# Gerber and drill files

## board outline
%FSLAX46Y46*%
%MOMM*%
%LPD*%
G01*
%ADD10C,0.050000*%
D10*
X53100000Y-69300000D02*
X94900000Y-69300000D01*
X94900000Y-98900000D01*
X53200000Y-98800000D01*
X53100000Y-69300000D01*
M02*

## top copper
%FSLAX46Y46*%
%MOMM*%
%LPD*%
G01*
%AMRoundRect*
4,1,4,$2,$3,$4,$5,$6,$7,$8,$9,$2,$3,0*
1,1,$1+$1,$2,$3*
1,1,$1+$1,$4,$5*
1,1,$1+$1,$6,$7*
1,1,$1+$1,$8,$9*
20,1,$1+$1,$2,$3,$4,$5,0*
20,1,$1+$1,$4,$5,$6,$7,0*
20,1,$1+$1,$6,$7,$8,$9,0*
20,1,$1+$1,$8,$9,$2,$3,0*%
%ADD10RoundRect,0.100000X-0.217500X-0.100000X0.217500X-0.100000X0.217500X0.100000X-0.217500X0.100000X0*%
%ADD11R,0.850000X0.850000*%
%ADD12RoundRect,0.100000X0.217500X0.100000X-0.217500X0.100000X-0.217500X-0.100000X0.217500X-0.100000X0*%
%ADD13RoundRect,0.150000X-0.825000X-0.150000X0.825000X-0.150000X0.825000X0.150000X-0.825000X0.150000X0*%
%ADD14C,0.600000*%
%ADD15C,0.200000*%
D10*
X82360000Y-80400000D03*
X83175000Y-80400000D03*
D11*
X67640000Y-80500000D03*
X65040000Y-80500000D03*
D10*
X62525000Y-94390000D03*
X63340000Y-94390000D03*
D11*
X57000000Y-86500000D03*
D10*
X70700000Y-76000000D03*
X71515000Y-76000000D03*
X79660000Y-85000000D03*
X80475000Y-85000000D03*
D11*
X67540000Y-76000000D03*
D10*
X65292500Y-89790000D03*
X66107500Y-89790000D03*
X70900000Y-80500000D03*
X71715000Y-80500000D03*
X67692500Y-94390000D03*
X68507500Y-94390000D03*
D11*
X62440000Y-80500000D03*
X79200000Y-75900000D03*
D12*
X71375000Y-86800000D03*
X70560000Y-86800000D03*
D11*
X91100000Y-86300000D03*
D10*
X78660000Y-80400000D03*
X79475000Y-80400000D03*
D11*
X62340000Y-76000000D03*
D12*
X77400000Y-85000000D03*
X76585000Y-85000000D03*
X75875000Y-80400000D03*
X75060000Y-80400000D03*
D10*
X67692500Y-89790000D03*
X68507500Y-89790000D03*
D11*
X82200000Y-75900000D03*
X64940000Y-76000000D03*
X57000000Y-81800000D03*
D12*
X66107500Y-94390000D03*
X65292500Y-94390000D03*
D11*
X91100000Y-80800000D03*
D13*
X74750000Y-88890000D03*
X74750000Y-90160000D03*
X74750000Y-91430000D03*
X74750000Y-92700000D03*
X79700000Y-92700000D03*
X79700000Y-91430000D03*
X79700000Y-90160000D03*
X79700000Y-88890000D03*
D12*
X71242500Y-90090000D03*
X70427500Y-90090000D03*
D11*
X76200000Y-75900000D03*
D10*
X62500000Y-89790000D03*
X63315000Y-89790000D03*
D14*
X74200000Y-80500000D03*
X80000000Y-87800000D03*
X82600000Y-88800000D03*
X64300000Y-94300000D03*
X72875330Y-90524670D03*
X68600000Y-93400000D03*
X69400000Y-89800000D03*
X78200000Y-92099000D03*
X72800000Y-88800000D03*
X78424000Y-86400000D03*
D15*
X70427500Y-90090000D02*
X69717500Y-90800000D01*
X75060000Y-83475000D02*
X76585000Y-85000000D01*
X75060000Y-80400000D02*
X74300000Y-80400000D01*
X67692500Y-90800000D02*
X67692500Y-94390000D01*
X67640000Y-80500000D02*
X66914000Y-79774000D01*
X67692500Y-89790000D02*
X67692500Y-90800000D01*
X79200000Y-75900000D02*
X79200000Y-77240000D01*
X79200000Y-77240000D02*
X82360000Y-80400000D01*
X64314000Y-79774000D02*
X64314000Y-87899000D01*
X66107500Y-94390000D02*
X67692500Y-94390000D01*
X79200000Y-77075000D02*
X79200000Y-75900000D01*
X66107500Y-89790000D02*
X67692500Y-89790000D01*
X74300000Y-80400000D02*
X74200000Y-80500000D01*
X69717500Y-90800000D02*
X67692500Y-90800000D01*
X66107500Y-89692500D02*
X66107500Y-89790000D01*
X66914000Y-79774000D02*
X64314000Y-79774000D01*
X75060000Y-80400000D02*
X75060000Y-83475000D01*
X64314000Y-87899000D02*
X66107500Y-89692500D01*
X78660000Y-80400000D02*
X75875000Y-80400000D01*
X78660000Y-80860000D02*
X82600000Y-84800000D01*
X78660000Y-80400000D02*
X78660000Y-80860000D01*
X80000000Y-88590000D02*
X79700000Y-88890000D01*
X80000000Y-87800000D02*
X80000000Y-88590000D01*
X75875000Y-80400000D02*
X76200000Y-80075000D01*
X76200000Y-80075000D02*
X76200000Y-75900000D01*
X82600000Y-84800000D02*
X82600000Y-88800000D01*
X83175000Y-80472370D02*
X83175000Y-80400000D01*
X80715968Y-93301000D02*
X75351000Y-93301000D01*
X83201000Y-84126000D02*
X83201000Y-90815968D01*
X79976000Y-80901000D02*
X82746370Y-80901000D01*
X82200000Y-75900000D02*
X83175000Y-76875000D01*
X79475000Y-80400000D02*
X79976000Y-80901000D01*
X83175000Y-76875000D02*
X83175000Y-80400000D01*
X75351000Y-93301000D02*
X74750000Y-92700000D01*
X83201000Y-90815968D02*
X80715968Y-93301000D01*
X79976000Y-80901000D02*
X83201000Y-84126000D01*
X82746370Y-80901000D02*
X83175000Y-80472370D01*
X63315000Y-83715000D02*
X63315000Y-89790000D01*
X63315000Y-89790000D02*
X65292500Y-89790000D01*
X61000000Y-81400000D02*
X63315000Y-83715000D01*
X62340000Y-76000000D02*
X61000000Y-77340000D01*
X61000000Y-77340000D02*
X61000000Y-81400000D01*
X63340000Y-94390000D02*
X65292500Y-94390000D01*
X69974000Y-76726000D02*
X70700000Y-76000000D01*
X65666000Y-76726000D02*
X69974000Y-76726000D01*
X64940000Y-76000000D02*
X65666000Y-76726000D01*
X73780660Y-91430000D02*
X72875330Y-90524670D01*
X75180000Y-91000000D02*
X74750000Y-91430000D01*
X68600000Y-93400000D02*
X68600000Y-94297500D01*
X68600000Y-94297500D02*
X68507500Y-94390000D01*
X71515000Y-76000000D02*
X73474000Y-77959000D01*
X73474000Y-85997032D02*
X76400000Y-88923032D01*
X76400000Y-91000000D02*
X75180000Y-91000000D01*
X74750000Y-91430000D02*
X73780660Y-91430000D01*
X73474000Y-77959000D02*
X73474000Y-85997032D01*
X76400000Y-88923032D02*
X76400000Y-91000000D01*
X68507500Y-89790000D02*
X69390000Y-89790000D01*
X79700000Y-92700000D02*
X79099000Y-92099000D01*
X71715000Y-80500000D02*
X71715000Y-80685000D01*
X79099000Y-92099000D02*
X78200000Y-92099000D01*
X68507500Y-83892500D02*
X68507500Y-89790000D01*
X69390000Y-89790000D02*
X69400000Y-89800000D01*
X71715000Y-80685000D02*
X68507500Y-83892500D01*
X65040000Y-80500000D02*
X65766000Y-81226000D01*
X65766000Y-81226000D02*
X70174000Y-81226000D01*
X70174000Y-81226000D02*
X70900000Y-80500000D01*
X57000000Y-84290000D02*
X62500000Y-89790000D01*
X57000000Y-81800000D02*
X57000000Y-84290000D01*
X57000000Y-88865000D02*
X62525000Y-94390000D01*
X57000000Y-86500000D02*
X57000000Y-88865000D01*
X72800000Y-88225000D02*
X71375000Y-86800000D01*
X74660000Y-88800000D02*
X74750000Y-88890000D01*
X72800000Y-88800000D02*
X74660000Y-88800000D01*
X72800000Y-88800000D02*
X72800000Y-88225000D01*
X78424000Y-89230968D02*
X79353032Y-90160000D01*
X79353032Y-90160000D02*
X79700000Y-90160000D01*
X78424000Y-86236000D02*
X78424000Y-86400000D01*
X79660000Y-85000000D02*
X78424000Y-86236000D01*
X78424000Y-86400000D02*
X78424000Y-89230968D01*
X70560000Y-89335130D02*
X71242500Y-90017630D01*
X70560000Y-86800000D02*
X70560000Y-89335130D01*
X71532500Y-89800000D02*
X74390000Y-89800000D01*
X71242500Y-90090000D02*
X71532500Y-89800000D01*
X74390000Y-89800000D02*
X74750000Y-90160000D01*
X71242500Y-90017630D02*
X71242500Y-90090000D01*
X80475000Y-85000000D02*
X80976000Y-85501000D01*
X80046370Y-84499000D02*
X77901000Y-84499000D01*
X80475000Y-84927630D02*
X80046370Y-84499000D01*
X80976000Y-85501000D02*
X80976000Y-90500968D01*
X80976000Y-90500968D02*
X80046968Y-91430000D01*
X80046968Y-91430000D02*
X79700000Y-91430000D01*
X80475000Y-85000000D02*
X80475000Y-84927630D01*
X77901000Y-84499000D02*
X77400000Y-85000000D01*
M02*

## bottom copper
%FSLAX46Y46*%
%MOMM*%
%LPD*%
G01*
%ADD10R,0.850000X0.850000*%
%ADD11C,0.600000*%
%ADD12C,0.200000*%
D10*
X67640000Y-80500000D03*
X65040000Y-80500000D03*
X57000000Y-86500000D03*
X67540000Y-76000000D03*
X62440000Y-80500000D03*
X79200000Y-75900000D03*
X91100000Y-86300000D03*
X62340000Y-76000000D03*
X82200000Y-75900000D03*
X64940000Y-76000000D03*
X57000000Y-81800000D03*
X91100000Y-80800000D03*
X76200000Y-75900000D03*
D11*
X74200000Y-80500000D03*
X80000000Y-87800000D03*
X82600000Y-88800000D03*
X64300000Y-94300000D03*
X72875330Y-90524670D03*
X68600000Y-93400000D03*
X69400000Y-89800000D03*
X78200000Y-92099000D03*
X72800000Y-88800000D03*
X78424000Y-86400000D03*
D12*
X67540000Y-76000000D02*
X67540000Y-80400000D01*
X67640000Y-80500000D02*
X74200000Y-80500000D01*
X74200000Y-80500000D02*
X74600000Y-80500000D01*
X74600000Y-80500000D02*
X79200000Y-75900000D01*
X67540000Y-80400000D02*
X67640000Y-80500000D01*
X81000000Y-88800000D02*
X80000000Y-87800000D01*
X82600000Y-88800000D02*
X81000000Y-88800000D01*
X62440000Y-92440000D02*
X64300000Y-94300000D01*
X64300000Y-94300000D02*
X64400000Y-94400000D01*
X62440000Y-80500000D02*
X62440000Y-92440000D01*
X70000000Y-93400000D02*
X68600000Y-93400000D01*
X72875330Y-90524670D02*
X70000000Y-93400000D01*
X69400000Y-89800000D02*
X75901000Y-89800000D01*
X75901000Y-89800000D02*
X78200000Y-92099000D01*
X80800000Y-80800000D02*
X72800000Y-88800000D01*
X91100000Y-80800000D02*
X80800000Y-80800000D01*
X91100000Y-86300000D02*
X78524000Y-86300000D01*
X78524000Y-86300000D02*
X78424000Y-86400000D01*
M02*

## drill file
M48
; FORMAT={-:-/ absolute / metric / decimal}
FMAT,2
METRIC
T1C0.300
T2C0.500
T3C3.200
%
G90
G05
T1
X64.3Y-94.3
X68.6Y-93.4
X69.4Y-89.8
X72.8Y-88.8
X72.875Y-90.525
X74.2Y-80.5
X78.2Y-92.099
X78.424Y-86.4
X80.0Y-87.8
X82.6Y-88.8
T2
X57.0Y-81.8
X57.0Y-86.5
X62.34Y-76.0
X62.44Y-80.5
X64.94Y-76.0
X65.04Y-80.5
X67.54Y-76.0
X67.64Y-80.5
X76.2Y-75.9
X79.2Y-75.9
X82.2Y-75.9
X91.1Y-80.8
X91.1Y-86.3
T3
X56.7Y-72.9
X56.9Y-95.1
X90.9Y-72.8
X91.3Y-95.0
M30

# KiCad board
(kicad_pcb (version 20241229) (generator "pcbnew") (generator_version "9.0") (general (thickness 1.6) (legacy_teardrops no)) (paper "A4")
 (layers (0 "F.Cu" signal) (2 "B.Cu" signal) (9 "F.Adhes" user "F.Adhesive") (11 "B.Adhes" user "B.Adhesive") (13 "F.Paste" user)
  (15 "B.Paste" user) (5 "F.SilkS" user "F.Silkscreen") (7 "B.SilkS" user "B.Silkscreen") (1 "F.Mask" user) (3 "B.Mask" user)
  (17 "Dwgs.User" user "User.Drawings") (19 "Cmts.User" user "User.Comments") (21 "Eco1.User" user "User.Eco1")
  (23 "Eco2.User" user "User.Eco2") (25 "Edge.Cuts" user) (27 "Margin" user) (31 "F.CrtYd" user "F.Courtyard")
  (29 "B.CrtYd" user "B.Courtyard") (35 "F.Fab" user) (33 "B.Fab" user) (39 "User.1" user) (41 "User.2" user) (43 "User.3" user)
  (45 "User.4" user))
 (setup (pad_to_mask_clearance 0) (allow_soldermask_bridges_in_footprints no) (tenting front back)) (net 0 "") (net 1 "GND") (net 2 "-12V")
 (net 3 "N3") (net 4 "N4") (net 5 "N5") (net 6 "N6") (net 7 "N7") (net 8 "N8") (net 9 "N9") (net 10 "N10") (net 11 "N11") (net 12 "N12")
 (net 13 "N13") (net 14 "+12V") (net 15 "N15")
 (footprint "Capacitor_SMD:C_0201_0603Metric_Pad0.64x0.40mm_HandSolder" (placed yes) (layer "F.Cu") (at 82.7675 80.4)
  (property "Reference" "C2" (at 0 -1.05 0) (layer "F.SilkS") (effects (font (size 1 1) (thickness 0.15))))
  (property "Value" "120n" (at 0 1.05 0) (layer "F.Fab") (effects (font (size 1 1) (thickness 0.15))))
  (pad "" smd roundrect (at -0.4325 0) (size 0.458 0.36) (layers "F.Paste") (roundrect_rratio 0.25))
  (pad "" smd roundrect (at 0.4325 0) (size 0.458 0.36) (layers "F.Paste") (roundrect_rratio 0.25))
  (pad "1" smd roundrect (at -0.4075 0) (size 0.635 0.4) (layers "F.Cu" "F.Mask") (roundrect_rratio 0.25) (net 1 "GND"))
  (pad "2" smd roundrect (at 0.4075 0) (size 0.635 0.4) (layers "F.Cu" "F.Mask") (roundrect_rratio 0.25) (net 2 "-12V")))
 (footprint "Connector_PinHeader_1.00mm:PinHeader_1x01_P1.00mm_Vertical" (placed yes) (layer "F.Cu") (at 67.64 80.5)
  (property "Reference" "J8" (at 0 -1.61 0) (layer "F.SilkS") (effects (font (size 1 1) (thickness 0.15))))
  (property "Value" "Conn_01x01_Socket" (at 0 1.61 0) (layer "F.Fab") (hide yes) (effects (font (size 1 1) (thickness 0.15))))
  (pad "1" thru_hole rect (at 0 0) (size 0.85 0.85) (drill 0.5) (layers "*.Cu" "*.Mask") (remove_unused_layers no) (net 1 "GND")))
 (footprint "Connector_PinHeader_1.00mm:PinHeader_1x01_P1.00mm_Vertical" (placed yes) (layer "F.Cu") (at 65.04 80.5)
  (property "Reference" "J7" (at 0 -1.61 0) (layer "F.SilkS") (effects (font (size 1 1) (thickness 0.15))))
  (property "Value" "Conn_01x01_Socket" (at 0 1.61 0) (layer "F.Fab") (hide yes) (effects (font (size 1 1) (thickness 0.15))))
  (pad "1" thru_hole rect (at 0 0) (size 0.85 0.85) (drill 0.5) (layers "*.Cu" "*.Mask") (remove_unused_layers no) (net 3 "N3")))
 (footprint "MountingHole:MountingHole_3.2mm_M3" (layer "F.Cu") (at 91.3 95)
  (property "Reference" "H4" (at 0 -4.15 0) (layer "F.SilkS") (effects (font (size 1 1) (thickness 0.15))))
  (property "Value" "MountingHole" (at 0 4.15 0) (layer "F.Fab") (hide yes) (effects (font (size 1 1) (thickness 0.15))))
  (pad "" np_thru_hole circle (at 0 0) (size 3.2 3.2) (drill 3.2) (layers "*.Cu" "*.Mask")))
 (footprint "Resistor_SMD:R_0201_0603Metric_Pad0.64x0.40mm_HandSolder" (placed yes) (layer "F.Cu") (at 62.9325 94.39)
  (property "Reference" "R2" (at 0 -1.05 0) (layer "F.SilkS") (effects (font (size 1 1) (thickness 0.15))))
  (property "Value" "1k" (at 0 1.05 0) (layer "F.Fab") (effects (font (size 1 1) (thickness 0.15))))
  (pad "" smd roundrect (at -0.4325 0) (size 0.458 0.36) (layers "F.Paste") (roundrect_rratio 0.25))
  (pad "" smd roundrect (at 0.4325 0) (size 0.458 0.36) (layers "F.Paste") (roundrect_rratio 0.25))
  (pad "1" smd roundrect (at -0.4075 0) (size 0.635 0.4) (layers "F.Cu" "F.Mask") (roundrect_rratio 0.25) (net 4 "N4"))
  (pad "2" smd roundrect (at 0.4075 0) (size 0.635 0.4) (layers "F.Cu" "F.Mask") (roundrect_rratio 0.25) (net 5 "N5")))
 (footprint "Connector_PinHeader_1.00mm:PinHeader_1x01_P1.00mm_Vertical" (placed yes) (layer "F.Cu") (at 57 86.5)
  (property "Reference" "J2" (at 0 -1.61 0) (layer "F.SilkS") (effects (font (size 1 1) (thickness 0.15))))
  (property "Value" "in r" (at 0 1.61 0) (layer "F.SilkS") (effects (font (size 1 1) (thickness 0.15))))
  (pad "1" thru_hole rect (at 0 0) (size 0.85 0.85) (drill 0.5) (layers "*.Cu" "*.Mask") (remove_unused_layers no) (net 4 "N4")))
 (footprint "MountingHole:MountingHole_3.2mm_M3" (layer "F.Cu") (at 56.7 72.9)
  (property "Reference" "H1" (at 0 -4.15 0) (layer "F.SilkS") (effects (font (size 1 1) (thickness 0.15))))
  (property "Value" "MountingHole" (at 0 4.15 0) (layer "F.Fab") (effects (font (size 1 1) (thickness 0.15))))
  (pad "" np_thru_hole circle (at 0 0) (size 3.2 3.2) (drill 3.2) (layers "*.Cu" "*.Mask")))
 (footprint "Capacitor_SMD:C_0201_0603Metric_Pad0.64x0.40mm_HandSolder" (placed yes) (layer "F.Cu") (at 71.1075 76)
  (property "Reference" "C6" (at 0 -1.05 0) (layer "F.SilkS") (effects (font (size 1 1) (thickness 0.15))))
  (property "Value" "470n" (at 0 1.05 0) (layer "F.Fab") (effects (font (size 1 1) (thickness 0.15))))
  (pad "" smd roundrect (at -0.4325 0) (size 0.458 0.36) (layers "F.Paste") (roundrect_rratio 0.25))
  (pad "" smd roundrect (at 0.4325 0) (size 0.458 0.36) (layers "F.Paste") (roundrect_rratio 0.25))
  (pad "1" smd roundrect (at -0.4075 0) (size 0.635 0.4) (layers "F.Cu" "F.Mask") (roundrect_rratio 0.25) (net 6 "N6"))
  (pad "2" smd roundrect (at 0.4075 0) (size 0.635 0.4) (layers "F.Cu" "F.Mask") (roundrect_rratio 0.25) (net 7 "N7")))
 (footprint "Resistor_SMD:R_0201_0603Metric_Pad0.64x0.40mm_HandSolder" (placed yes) (layer "F.Cu") (at 80.0675 85)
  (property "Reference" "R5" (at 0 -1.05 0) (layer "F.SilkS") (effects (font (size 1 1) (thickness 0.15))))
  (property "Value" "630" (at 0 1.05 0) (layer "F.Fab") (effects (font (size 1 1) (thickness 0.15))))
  (pad "" smd roundrect (at -0.4325 0) (size 0.458 0.36) (layers "F.Paste") (roundrect_rratio 0.25))
  (pad "" smd roundrect (at 0.4325 0) (size 0.458 0.36) (layers "F.Paste") (roundrect_rratio 0.25))
  (pad "1" smd roundrect (at -0.4075 0) (size 0.635 0.4) (layers "F.Cu" "F.Mask") (roundrect_rratio 0.25) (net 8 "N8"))
  (pad "2" smd roundrect (at 0.4075 0) (size 0.635 0.4) (layers "F.Cu" "F.Mask") (roundrect_rratio 0.25) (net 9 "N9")))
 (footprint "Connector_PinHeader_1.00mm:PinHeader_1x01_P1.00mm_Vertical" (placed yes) (layer "F.Cu") (at 67.54 76)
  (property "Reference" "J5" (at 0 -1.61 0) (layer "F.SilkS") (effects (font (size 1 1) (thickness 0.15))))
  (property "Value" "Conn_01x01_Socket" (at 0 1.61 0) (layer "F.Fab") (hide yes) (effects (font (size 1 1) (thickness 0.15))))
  (pad "1" thru_hole rect (at 0 0) (size 0.85 0.85) (drill 0.5) (layers "*.Cu" "*.Mask") (remove_unused_layers no) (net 1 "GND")))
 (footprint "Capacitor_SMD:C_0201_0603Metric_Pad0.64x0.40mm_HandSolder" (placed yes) (layer "F.Cu") (at 65.7 89.79)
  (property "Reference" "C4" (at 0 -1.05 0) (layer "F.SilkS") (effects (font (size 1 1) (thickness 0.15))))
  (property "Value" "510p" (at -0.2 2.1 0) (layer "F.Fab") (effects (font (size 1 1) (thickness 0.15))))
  (pad "" smd roundrect (at -0.4325 0) (size 0.458 0.36) (layers "F.Paste") (roundrect_rratio 0.25))
  (pad "" smd roundrect (at 0.4325 0) (size 0.458 0.36) (layers "F.Paste") (roundrect_rratio 0.25))
  (pad "1" smd roundrect (at -0.4075 0) (size 0.635 0.4) (layers "F.Cu" "F.Mask") (roundrect_rratio 0.25) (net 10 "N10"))
  (pad "2" smd roundrect (at 0.4075 0) (size 0.635 0.4) (layers "F.Cu" "F.Mask") (roundrect_rratio 0.25) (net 1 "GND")))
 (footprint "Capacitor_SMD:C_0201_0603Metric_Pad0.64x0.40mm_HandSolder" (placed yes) (layer "F.Cu") (at 71.3075 80.5)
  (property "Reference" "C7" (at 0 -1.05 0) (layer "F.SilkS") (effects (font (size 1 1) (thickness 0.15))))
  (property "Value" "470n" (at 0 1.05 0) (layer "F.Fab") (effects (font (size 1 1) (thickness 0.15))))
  (pad "" smd roundrect (at -0.4325 0) (size 0.458 0.36) (layers "F.Paste") (roundrect_rratio 0.25))
  (pad "" smd roundrect (at 0.4325 0) (size 0.458 0.36) (layers "F.Paste") (roundrect_rratio 0.25))
  (pad "1" smd roundrect (at -0.4075 0) (size 0.635 0.4) (layers "F.Cu" "F.Mask") (roundrect_rratio 0.25) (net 3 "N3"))
  (pad "2" smd roundrect (at 0.4075 0) (size 0.635 0.4) (layers "F.Cu" "F.Mask") (roundrect_rratio 0.25) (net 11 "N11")))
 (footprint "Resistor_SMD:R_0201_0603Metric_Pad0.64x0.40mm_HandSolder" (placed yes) (layer "F.Cu") (at 68.1 94.39)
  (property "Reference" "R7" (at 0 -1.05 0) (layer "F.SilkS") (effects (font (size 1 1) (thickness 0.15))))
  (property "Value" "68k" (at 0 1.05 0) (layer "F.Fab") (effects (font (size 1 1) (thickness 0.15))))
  (pad "" smd roundrect (at -0.4325 0) (size 0.458 0.36) (layers "F.Paste") (roundrect_rratio 0.25))
  (pad "" smd roundrect (at 0.4325 0) (size 0.458 0.36) (layers "F.Paste") (roundrect_rratio 0.25))
  (pad "1" smd roundrect (at -0.4075 0) (size 0.635 0.4) (layers "F.Cu" "F.Mask") (roundrect_rratio 0.25) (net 1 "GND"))
  (pad "2" smd roundrect (at 0.4075 0) (size 0.635 0.4) (layers "F.Cu" "F.Mask") (roundrect_rratio 0.25) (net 7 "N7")))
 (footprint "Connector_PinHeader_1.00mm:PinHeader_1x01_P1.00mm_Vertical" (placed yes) (layer "F.Cu") (at 62.44 80.5)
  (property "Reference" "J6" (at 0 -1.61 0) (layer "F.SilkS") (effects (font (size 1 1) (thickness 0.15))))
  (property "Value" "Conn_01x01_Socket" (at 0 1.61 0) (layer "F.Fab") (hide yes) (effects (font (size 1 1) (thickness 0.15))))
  (pad "1" thru_hole rect (at 0 0) (size 0.85 0.85) (drill 0.5) (layers "*.Cu" "*.Mask") (remove_unused_layers no) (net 5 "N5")))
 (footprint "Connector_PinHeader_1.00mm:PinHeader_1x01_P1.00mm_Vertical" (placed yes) (layer "F.Cu") (at 79.2 75.9)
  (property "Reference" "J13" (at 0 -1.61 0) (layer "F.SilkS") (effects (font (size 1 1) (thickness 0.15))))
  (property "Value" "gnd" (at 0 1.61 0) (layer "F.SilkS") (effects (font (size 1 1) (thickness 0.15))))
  (pad "1" thru_hole rect (at 0 0) (size 0.85 0.85) (drill 0.5) (layers "*.Cu" "*.Mask") (remove_unused_layers no) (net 1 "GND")))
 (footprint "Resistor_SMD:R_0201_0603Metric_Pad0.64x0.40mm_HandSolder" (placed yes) (layer "F.Cu") (at 70.9675 86.8 180)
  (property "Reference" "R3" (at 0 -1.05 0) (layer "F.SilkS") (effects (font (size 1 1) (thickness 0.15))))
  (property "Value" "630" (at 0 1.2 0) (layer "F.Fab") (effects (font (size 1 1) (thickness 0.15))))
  (pad "" smd roundrect (at -0.4325 0 180) (size 0.458 0.36) (layers "F.Paste") (roundrect_rratio 0.25))
  (pad "" smd roundrect (at 0.4325 0 180) (size 0.458 0.36) (layers "F.Paste") (roundrect_rratio 0.25))
  (pad "1" smd roundrect (at -0.4075 0 180) (size 0.635 0.4) (layers "F.Cu" "F.Mask") (roundrect_rratio 0.25) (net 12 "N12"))
  (pad "2" smd roundrect (at 0.4075 0 180) (size 0.635 0.4) (layers "F.Cu" "F.Mask") (roundrect_rratio 0.25) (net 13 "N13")))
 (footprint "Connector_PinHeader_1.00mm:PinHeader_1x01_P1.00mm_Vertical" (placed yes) (layer "F.Cu") (at 91.1 86.3)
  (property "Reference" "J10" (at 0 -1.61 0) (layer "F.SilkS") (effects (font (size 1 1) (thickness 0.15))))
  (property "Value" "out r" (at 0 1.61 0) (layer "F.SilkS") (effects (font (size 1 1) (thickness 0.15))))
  (pad "1" thru_hole rect (at 0 0) (size 0.85 0.85) (drill 0.5) (layers "*.Cu" "*.Mask") (remove_unused_layers no) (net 8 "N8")))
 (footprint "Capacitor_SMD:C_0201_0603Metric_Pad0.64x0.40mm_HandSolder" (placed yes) (layer "F.Cu") (at 79.0675 80.4)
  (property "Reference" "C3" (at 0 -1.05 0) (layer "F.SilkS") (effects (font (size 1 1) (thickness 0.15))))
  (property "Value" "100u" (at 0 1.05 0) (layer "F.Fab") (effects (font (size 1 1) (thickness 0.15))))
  (pad "" smd roundrect (at -0.4325 0) (size 0.458 0.36) (layers "F.Paste") (roundrect_rratio 0.25))
  (pad "" smd roundrect (at 0.4325 0) (size 0.458 0.36) (layers "F.Paste") (roundrect_rratio 0.25))
  (pad "1" smd roundrect (at -0.4075 0) (size 0.635 0.4) (layers "F.Cu" "F.Mask") (roundrect_rratio 0.25) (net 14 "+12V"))
  (pad "2" smd roundrect (at 0.4075 0) (size 0.635 0.4) (layers "F.Cu" "F.Mask") (roundrect_rratio 0.25) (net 2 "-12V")))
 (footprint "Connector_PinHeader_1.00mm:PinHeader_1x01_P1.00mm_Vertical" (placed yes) (layer "F.Cu") (at 62.34 76)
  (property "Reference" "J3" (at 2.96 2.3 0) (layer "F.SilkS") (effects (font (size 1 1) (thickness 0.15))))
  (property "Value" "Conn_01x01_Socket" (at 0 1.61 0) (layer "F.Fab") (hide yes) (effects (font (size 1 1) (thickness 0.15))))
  (pad "1" thru_hole rect (at 0 0) (size 0.85 0.85) (drill 0.5) (layers "*.Cu" "*.Mask") (remove_unused_layers no) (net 10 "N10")))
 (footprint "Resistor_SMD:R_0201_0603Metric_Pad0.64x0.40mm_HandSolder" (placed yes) (layer "F.Cu") (at 76.9925 85 180)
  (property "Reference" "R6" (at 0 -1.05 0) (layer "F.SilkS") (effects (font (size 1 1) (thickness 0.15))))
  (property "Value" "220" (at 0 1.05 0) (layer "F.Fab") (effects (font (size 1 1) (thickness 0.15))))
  (pad "" smd roundrect (at -0.4325 0 180) (size 0.458 0.36) (layers "F.Paste") (roundrect_rratio 0.25))
  (pad "" smd roundrect (at 0.4325 0 180) (size 0.458 0.36) (layers "F.Paste") (roundrect_rratio 0.25))
  (pad "1" smd roundrect (at -0.4075 0 180) (size 0.635 0.4) (layers "F.Cu" "F.Mask") (roundrect_rratio 0.25) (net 9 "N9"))
  (pad "2" smd roundrect (at 0.4075 0 180) (size 0.635 0.4) (layers "F.Cu" "F.Mask") (roundrect_rratio 0.25) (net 1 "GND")))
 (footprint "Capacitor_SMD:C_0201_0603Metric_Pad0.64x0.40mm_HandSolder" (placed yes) (layer "F.Cu") (at 75.4675 80.4 180)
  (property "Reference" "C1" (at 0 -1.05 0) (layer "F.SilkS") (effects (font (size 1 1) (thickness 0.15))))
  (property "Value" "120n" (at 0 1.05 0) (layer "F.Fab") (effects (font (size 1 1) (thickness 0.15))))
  (pad "" smd roundrect (at -0.4325 0 180) (size 0.458 0.36) (layers "F.Paste") (roundrect_rratio 0.25))
  (pad "" smd roundrect (at 0.4325 0 180) (size 0.458 0.36) (layers "F.Paste") (roundrect_rratio 0.25))
  (pad "1" smd roundrect (at -0.4075 0 180) (size 0.635 0.4) (layers "F.Cu" "F.Mask") (roundrect_rratio 0.25) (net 14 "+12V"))
  (pad "2" smd roundrect (at 0.4075 0 180) (size 0.635 0.4) (layers "F.Cu" "F.Mask") (roundrect_rratio 0.25) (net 1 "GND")))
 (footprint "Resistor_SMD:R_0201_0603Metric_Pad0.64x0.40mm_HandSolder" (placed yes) (layer "F.Cu") (at 68.1 89.79)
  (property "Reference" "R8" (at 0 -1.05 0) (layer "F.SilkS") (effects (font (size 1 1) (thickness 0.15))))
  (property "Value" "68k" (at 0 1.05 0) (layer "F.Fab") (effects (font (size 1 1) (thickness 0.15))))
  (pad "" smd roundrect (at -0.4325 0) (size 0.458 0.36) (layers "F.Paste") (roundrect_rratio 0.25))
  (pad "" smd roundrect (at 0.4325 0) (size 0.458 0.36) (layers "F.Paste") (roundrect_rratio 0.25))
  (pad "1" smd roundrect (at -0.4075 0) (size 0.635 0.4) (layers "F.Cu" "F.Mask") (roundrect_rratio 0.25) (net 1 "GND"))
  (pad "2" smd roundrect (at 0.4075 0) (size 0.635 0.4) (layers "F.Cu" "F.Mask") (roundrect_rratio 0.25) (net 11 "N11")))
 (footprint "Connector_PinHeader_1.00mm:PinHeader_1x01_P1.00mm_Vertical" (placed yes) (layer "F.Cu") (at 82.2 75.9)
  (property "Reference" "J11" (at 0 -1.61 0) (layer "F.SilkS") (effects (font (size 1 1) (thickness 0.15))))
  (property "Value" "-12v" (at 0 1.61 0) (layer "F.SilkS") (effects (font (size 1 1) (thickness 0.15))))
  (pad "1" thru_hole rect (at 0 0) (size 0.85 0.85) (drill 0.5) (layers "*.Cu" "*.Mask") (remove_unused_layers no) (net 2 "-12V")))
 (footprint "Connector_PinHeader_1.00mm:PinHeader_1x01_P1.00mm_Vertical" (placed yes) (layer "F.Cu") (at 64.94 76)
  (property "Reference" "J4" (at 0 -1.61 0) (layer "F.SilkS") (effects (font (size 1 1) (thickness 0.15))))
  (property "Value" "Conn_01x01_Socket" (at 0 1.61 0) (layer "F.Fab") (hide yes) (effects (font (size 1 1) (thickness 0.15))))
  (pad "1" thru_hole rect (at 0 0) (size 0.85 0.85) (drill 0.5) (layers "*.Cu" "*.Mask") (remove_unused_layers no) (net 6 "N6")))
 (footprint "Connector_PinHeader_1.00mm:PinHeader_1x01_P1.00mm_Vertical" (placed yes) (layer "F.Cu") (at 57 81.8)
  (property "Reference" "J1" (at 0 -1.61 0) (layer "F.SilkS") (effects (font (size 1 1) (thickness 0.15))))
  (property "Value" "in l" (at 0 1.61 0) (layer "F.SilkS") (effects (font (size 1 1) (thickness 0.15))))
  (pad "1" thru_hole rect (at 0 0) (size 0.85 0.85) (drill 0.5) (layers "*.Cu" "*.Mask") (remove_unused_layers no) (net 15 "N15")))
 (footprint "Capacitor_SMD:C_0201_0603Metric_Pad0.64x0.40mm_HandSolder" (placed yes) (layer "F.Cu") (at 65.7 94.39 180)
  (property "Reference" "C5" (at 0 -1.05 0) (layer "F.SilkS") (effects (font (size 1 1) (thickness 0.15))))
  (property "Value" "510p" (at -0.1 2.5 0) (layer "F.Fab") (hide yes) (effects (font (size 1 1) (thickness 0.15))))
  (pad "" smd roundrect (at -0.4325 0 180) (size 0.458 0.36) (layers "F.Paste") (roundrect_rratio 0.25))
  (pad "" smd roundrect (at 0.4325 0 180) (size 0.458 0.36) (layers "F.Paste") (roundrect_rratio 0.25))
  (pad "1" smd roundrect (at -0.4075 0 180) (size 0.635 0.4) (layers "F.Cu" "F.Mask") (roundrect_rratio 0.25) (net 1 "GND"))
  (pad "2" smd roundrect (at 0.4075 0 180) (size 0.635 0.4) (layers "F.Cu" "F.Mask") (roundrect_rratio 0.25) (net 5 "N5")))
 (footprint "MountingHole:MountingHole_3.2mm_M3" (layer "F.Cu") (at 56.9 95.1)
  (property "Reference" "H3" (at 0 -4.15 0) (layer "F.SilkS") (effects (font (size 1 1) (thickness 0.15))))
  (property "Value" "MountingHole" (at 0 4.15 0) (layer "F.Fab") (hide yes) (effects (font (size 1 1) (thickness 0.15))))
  (pad "" np_thru_hole circle (at 0 0) (size 3.2 3.2) (drill 3.2) (layers "*.Cu" "*.Mask")))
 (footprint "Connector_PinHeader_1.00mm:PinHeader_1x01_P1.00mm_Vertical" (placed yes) (layer "F.Cu") (at 91.1 80.8)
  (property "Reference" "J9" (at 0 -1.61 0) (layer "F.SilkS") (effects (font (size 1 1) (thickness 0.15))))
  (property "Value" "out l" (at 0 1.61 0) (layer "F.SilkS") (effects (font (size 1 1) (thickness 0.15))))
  (pad "1" thru_hole rect (at 0 0) (size 0.85 0.85) (drill 0.5) (layers "*.Cu" "*.Mask") (remove_unused_layers no) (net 12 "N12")))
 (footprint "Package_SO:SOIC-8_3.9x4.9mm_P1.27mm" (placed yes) (layer "F.Cu") (at 77.225 90.795)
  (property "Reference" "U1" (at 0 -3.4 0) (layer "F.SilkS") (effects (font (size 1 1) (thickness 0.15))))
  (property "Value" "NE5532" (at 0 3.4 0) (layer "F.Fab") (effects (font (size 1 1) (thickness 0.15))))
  (pad "1" smd roundrect (at -2.475 -1.905) (size 1.95 0.6) (layers "F.Cu" "F.Mask" "F.Paste") (roundrect_rratio 0.25) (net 12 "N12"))
  (pad "2" smd roundrect (at -2.475 -0.635) (size 1.95 0.6) (layers "F.Cu" "F.Mask" "F.Paste") (roundrect_rratio 0.25) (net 13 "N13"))
  (pad "3" smd roundrect (at -2.475 0.635) (size 1.95 0.6) (layers "F.Cu" "F.Mask" "F.Paste") (roundrect_rratio 0.25) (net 7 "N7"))
  (pad "4" smd roundrect (at -2.475 1.905) (size 1.95 0.6) (layers "F.Cu" "F.Mask" "F.Paste") (roundrect_rratio 0.25) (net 2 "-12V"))
  (pad "5" smd roundrect (at 2.475 1.905) (size 1.95 0.6) (layers "F.Cu" "F.Mask" "F.Paste") (roundrect_rratio 0.25) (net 11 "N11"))
  (pad "6" smd roundrect (at 2.475 0.635) (size 1.95 0.6) (layers "F.Cu" "F.Mask" "F.Paste") (roundrect_rratio 0.25) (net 9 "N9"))
  (pad "7" smd roundrect (at 2.475 -0.635) (size 1.95 0.6) (layers "F.Cu" "F.Mask" "F.Paste") (roundrect_rratio 0.25) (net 8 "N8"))
  (pad "8" smd roundrect (at 2.475 -1.905) (size 1.95 0.6) (layers "F.Cu" "F.Mask" "F.Paste") (roundrect_rratio 0.25) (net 14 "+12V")))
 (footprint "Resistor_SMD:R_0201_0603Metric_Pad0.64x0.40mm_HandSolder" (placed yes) (layer "F.Cu") (at 70.835 90.09 180)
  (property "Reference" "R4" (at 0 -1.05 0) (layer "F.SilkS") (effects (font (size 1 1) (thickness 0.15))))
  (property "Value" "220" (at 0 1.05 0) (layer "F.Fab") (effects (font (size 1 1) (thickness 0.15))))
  (pad "" smd roundrect (at -0.4325 0 180) (size 0.458 0.36) (layers "F.Paste") (roundrect_rratio 0.25))
  (pad "" smd roundrect (at 0.4325 0 180) (size 0.458 0.36) (layers "F.Paste") (roundrect_rratio 0.25))
  (pad "1" smd roundrect (at -0.4075 0 180) (size 0.635 0.4) (layers "F.Cu" "F.Mask") (roundrect_rratio 0.25) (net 13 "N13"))
  (pad "2" smd roundrect (at 0.4075 0 180) (size 0.635 0.4) (layers "F.Cu" "F.Mask") (roundrect_rratio 0.25) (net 1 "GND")))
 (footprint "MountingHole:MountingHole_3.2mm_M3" (layer "F.Cu") (at 90.9 72.8)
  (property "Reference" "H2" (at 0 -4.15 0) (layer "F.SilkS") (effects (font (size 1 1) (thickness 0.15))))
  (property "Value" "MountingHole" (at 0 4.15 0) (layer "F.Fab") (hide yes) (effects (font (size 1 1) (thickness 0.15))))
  (pad "" np_thru_hole circle (at 0 0) (size 3.2 3.2) (drill 3.2) (layers "*.Cu" "*.Mask")))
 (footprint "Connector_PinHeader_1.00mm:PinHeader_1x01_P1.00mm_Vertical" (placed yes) (layer "F.Cu") (at 76.2 75.9)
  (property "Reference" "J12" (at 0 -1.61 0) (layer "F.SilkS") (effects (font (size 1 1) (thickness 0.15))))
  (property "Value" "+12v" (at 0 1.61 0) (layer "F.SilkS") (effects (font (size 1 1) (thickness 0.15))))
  (pad "1" thru_hole rect (at 0 0) (size 0.85 0.85) (drill 0.5) (layers "*.Cu" "*.Mask") (remove_unused_layers no) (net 14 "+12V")))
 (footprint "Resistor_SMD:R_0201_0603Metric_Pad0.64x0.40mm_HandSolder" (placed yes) (layer "F.Cu") (at 62.9075 89.79)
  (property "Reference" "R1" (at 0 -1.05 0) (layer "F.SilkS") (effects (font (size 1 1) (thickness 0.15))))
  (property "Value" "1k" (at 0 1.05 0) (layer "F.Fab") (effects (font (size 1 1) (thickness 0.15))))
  (pad "" smd roundrect (at -0.4325 0) (size 0.458 0.36) (layers "F.Paste") (roundrect_rratio 0.25))
  (pad "" smd roundrect (at 0.4325 0) (size 0.458 0.36) (layers "F.Paste") (roundrect_rratio 0.25))
  (pad "1" smd roundrect (at -0.4075 0) (size 0.635 0.4) (layers "F.Cu" "F.Mask") (roundrect_rratio 0.25) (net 15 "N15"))
  (pad "2" smd roundrect (at 0.4075 0) (size 0.635 0.4) (layers "F.Cu" "F.Mask") (roundrect_rratio 0.25) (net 10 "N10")))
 (gr_poly
  (pts (xy 53.1 69.3) (xy 94.9 69.3) (xy 94.9 98.9) (xy 53.2 98.8) (xy 53.1 69.3)) (stroke (width 0.05) (type solid)) (fill no)
  (layer "Edge.Cuts"))
 (segment (start 70.4275 90.09) (end 69.7175 90.8) (width 0.2) (layer "F.Cu") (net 1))
 (segment (start 75.06 83.475) (end 76.585 85) (width 0.2) (layer "F.Cu") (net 1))
 (segment (start 75.06 80.4) (end 74.3 80.4) (width 0.2) (layer "F.Cu") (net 1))
 (segment (start 67.6925 90.8) (end 67.6925 94.39) (width 0.2) (layer "F.Cu") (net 1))
 (segment (start 67.64 80.5) (end 66.914 79.774) (width 0.2) (layer "F.Cu") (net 1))
 (segment (start 67.6925 89.79) (end 67.6925 90.8) (width 0.2) (layer "F.Cu") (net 1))
 (segment (start 79.2 75.9) (end 79.2 77.24) (width 0.2) (layer "F.Cu") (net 1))
 (segment (start 79.2 77.24) (end 82.36 80.4) (width 0.2) (layer "F.Cu") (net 1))
 (segment (start 64.314 79.774) (end 64.314 87.899) (width 0.2) (layer "F.Cu") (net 1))
 (segment (start 66.1075 94.39) (end 67.6925 94.39) (width 0.2) (layer "F.Cu") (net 1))
 (segment (start 79.2 77.075) (end 79.2 75.9) (width 0.2) (layer "F.Cu") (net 1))
 (segment (start 66.1075 89.79) (end 67.6925 89.79) (width 0.2) (layer "F.Cu") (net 1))
 (segment (start 74.3 80.4) (end 74.2 80.5) (width 0.2) (layer "F.Cu") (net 1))
 (segment (start 69.7175 90.8) (end 67.6925 90.8) (width 0.2) (layer "F.Cu") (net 1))
 (segment (start 66.1075 89.6925) (end 66.1075 89.79) (width 0.2) (layer "F.Cu") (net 1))
 (segment (start 66.914 79.774) (end 64.314 79.774) (width 0.2) (layer "F.Cu") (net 1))
 (segment (start 75.06 80.4) (end 75.06 83.475) (width 0.2) (layer "F.Cu") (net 1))
 (segment (start 64.314 87.899) (end 66.1075 89.6925) (width 0.2) (layer "F.Cu") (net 1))
 (via (at 74.2 80.5) (size 0.6) (drill 0.3) (layers "F.Cu" "B.Cu") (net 1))
 (segment (start 67.54 76) (end 67.54 80.4) (width 0.2) (layer "B.Cu") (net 1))
 (segment (start 67.64 80.5) (end 74.2 80.5) (width 0.2) (layer "B.Cu") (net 1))
 (segment (start 74.2 80.5) (end 74.6 80.5) (width 0.2) (layer "B.Cu") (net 1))
 (segment (start 74.6 80.5) (end 79.2 75.9) (width 0.2) (layer "B.Cu") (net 1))
 (segment (start 67.54 80.4) (end 67.64 80.5) (width 0.2) (layer "B.Cu") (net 1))
 (segment (start 78.66 80.4) (end 75.875 80.4) (width 0.2) (layer "F.Cu") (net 14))
 (segment (start 78.66 80.86) (end 82.6 84.8) (width 0.2) (layer "F.Cu") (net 14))
 (segment (start 78.66 80.4) (end 78.66 80.86) (width 0.2) (layer "F.Cu") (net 14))
 (segment (start 80 88.59) (end 79.7 88.89) (width 0.2) (layer "F.Cu") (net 14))
 (segment (start 80 87.8) (end 80 88.59) (width 0.2) (layer "F.Cu") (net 14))
 (segment (start 75.875 80.4) (end 76.2 80.075) (width 0.2) (layer "F.Cu") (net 14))
 (segment (start 76.2 80.075) (end 76.2 75.9) (width 0.2) (layer "F.Cu") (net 14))
 (segment (start 82.6 84.8) (end 82.6 88.8) (width 0.2) (layer "F.Cu") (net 14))
 (via (at 80 87.8) (size 0.6) (drill 0.3) (layers "F.Cu" "B.Cu") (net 14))
 (via (at 82.6 88.8) (size 0.6) (drill 0.3) (layers "F.Cu" "B.Cu") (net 14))
 (segment (start 81 88.8) (end 80 87.8) (width 0.2) (layer "B.Cu") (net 14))
 (segment (start 82.6 88.8) (end 81 88.8) (width 0.2) (layer "B.Cu") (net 14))
 (segment (start 83.175 80.47237) (end 83.175 80.4) (width 0.2) (layer "F.Cu") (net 2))
 (segment (start 80.715968 93.301) (end 75.351 93.301) (width 0.2) (layer "F.Cu") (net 2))
 (segment (start 83.201 84.126) (end 83.201 90.815968) (width 0.2) (layer "F.Cu") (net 2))
 (segment (start 79.976 80.901) (end 82.74637 80.901) (width 0.2) (layer "F.Cu") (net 2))
 (segment (start 82.2 75.9) (end 83.175 76.875) (width 0.2) (layer "F.Cu") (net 2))
 (segment (start 79.475 80.4) (end 79.976 80.901) (width 0.2) (layer "F.Cu") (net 2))
 (segment (start 83.175 76.875) (end 83.175 80.4) (width 0.2) (layer "F.Cu") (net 2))
 (segment (start 75.351 93.301) (end 74.75 92.7) (width 0.2) (layer "F.Cu") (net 2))
 (segment (start 83.201 90.815968) (end 80.715968 93.301) (width 0.2) (layer "F.Cu") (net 2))
 (segment (start 79.976 80.901) (end 83.201 84.126) (width 0.2) (layer "F.Cu") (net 2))
 (segment (start 82.74637 80.901) (end 83.175 80.47237) (width 0.2) (layer "F.Cu") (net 2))
 (segment (start 63.315 83.715) (end 63.315 89.79) (width 0.2) (layer "F.Cu") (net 10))
 (segment (start 63.315 89.79) (end 65.2925 89.79) (width 0.2) (layer "F.Cu") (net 10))
 (segment (start 61 81.4) (end 63.315 83.715) (width 0.2) (layer "F.Cu") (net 10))
 (segment (start 62.34 76) (end 61 77.34) (width 0.2) (layer "F.Cu") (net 10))
 (segment (start 61 77.34) (end 61 81.4) (width 0.2) (layer "F.Cu") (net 10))
 (segment (start 63.34 94.39) (end 65.2925 94.39) (width 0.2) (layer "F.Cu") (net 5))
 (via (at 64.3 94.3) (size 0.6) (drill 0.3) (layers "F.Cu" "B.Cu") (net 5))
 (segment (start 62.44 92.44) (end 64.3 94.3) (width 0.2) (layer "B.Cu") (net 5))
 (segment (start 64.3 94.3) (end 64.4 94.4) (width 0.2) (layer "B.Cu") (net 5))
 (segment (start 62.44 80.5) (end 62.44 92.44) (width 0.2) (layer "B.Cu") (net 5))
 (segment (start 69.974 76.726) (end 70.7 76) (width 0.2) (layer "F.Cu") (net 6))
 (segment (start 65.666 76.726) (end 69.974 76.726) (width 0.2) (layer "F.Cu") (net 6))
 (segment (start 64.94 76) (end 65.666 76.726) (width 0.2) (layer "F.Cu") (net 6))
 (segment (start 73.78066 91.43) (end 72.87533 90.52467) (width 0.2) (layer "F.Cu") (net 7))
 (segment (start 75.18 91) (end 74.75 91.43) (width 0.2) (layer "F.Cu") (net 7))
 (segment (start 68.6 93.4) (end 68.6 94.2975) (width 0.2) (layer "F.Cu") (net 7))
 (segment (start 68.6 94.2975) (end 68.5075 94.39) (width 0.2) (layer "F.Cu") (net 7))
 (segment (start 71.515 76) (end 73.474 77.959) (width 0.2) (layer "F.Cu") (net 7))
 (segment (start 73.474 85.997032) (end 76.4 88.923032) (width 0.2) (layer "F.Cu") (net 7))
 (segment (start 76.4 91) (end 75.18 91) (width 0.2) (layer "F.Cu") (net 7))
 (segment (start 74.75 91.43) (end 73.78066 91.43) (width 0.2) (layer "F.Cu") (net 7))
 (segment (start 73.474 77.959) (end 73.474 85.997032) (width 0.2) (layer "F.Cu") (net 7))
 (segment (start 76.4 88.923032) (end 76.4 91) (width 0.2) (layer "F.Cu") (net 7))
 (via (at 72.87533 90.52467) (size 0.6) (drill 0.3) (layers "F.Cu" "B.Cu") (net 7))
 (via (at 68.6 93.4) (size 0.6) (drill 0.3) (layers "F.Cu" "B.Cu") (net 7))
 (segment (start 70 93.4) (end 68.6 93.4) (width 0.2) (layer "B.Cu") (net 7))
 (segment (start 72.87533 90.52467) (end 70 93.4) (width 0.2) (layer "B.Cu") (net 7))
 (segment (start 68.5075 89.79) (end 69.39 89.79) (width 0.2) (layer "F.Cu") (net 11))
 (segment (start 79.7 92.7) (end 79.099 92.099) (width 0.2) (layer "F.Cu") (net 11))
 (segment (start 71.715 80.5) (end 71.715 80.685) (width 0.2) (layer "F.Cu") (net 11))
 (segment (start 79.099 92.099) (end 78.2 92.099) (width 0.2) (layer "F.Cu") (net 11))
 (segment (start 68.5075 83.8925) (end 68.5075 89.79) (width 0.2) (layer "F.Cu") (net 11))
 (segment (start 69.39 89.79) (end 69.4 89.8) (width 0.2) (layer "F.Cu") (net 11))
 (segment (start 71.715 80.685) (end 68.5075 83.8925) (width 0.2) (layer "F.Cu") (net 11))
 (via (at 69.4 89.8) (size 0.6) (drill 0.3) (layers "F.Cu" "B.Cu") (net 11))
 (via (at 78.2 92.099) (size 0.6) (drill 0.3) (layers "F.Cu" "B.Cu") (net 11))
 (segment (start 69.4 89.8) (end 75.901 89.8) (width 0.2) (layer "B.Cu") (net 11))
 (segment (start 75.901 89.8) (end 78.2 92.099) (width 0.2) (layer "B.Cu") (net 11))
 (segment (start 65.04 80.5) (end 65.766 81.226) (width 0.2) (layer "F.Cu") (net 3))
 (segment (start 65.766 81.226) (end 70.174 81.226) (width 0.2) (layer "F.Cu") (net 3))
 (segment (start 70.174 81.226) (end 70.9 80.5) (width 0.2) (layer "F.Cu") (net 3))
 (segment (start 57 84.29) (end 62.5 89.79) (width 0.2) (layer "F.Cu") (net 15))
 (segment (start 57 81.8) (end 57 84.29) (width 0.2) (layer "F.Cu") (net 15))
 (segment (start 57 88.865) (end 62.525 94.39) (width 0.2) (layer "F.Cu") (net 4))
 (segment (start 57 86.5) (end 57 88.865) (width 0.2) (layer "F.Cu") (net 4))
 (segment (start 72.8 88.225) (end 71.375 86.8) (width 0.2) (layer "F.Cu") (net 12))
 (segment (start 74.66 88.8) (end 74.75 88.89) (width 0.2) (layer "F.Cu") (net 12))
 (segment (start 72.8 88.8) (end 74.66 88.8) (width 0.2) (layer "F.Cu") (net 12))
 (segment (start 72.8 88.8) (end 72.8 88.225) (width 0.2) (layer "F.Cu") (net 12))
 (via (at 72.8 88.8) (size 0.6) (drill 0.3) (layers "F.Cu" "B.Cu") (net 12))
 (segment (start 80.8 80.8) (end 72.8 88.8) (width 0.2) (layer "B.Cu") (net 12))
 (segment (start 91.1 80.8) (end 80.8 80.8) (width 0.2) (layer "B.Cu") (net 12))
 (segment (start 78.424 89.230968) (end 79.353032 90.16) (width 0.2) (layer "F.Cu") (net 8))
 (segment (start 79.353032 90.16) (end 79.7 90.16) (width 0.2) (layer "F.Cu") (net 8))
 (segment (start 78.424 86.236) (end 78.424 86.4) (width 0.2) (layer "F.Cu") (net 8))
 (segment (start 79.66 85) (end 78.424 86.236) (width 0.2) (layer "F.Cu") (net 8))
 (segment (start 78.424 86.4) (end 78.424 89.230968) (width 0.2) (layer "F.Cu") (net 8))
 (via (at 78.424 86.4) (size 0.6) (drill 0.3) (layers "F.Cu" "B.Cu") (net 8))
 (segment (start 91.1 86.3) (end 78.524 86.3) (width 0.2) (layer "B.Cu") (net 8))
 (segment (start 78.524 86.3) (end 78.424 86.4) (width 0.2) (layer "B.Cu") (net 8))
 (segment (start 70.56 89.33513) (end 71.2425 90.01763) (width 0.2) (layer "F.Cu") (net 13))
 (segment (start 70.56 86.8) (end 70.56 89.33513) (width 0.2) (layer "F.Cu") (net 13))
 (segment (start 71.5325 89.8) (end 74.39 89.8) (width 0.2) (layer "F.Cu") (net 13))
 (segment (start 71.2425 90.09) (end 71.5325 89.8) (width 0.2) (layer "F.Cu") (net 13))
 (segment (start 74.39 89.8) (end 74.75 90.16) (width 0.2) (layer "F.Cu") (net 13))
 (segment (start 71.2425 90.01763) (end 71.2425 90.09) (width 0.2) (layer "F.Cu") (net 13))
 (segment (start 80.475 85) (end 80.976 85.501) (width 0.2) (layer "F.Cu") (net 9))
 (segment (start 80.04637 84.499) (end 77.901 84.499) (width 0.2) (layer "F.Cu") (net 9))
 (segment (start 80.475 84.92763) (end 80.04637 84.499) (width 0.2) (layer "F.Cu") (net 9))
 (segment (start 80.976 85.501) (end 80.976 90.500968) (width 0.2) (layer "F.Cu") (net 9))
 (segment (start 80.976 90.500968) (end 80.046968 91.43) (width 0.2) (layer "F.Cu") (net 9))
 (segment (start 80.046968 91.43) (end 79.7 91.43) (width 0.2) (layer "F.Cu") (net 9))
 (segment (start 80.475 85) (end 80.475 84.92763) (width 0.2) (layer "F.Cu") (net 9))
 (segment (start 77.901 84.499) (end 77.4 85) (width 0.2) (layer "F.Cu") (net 9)))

